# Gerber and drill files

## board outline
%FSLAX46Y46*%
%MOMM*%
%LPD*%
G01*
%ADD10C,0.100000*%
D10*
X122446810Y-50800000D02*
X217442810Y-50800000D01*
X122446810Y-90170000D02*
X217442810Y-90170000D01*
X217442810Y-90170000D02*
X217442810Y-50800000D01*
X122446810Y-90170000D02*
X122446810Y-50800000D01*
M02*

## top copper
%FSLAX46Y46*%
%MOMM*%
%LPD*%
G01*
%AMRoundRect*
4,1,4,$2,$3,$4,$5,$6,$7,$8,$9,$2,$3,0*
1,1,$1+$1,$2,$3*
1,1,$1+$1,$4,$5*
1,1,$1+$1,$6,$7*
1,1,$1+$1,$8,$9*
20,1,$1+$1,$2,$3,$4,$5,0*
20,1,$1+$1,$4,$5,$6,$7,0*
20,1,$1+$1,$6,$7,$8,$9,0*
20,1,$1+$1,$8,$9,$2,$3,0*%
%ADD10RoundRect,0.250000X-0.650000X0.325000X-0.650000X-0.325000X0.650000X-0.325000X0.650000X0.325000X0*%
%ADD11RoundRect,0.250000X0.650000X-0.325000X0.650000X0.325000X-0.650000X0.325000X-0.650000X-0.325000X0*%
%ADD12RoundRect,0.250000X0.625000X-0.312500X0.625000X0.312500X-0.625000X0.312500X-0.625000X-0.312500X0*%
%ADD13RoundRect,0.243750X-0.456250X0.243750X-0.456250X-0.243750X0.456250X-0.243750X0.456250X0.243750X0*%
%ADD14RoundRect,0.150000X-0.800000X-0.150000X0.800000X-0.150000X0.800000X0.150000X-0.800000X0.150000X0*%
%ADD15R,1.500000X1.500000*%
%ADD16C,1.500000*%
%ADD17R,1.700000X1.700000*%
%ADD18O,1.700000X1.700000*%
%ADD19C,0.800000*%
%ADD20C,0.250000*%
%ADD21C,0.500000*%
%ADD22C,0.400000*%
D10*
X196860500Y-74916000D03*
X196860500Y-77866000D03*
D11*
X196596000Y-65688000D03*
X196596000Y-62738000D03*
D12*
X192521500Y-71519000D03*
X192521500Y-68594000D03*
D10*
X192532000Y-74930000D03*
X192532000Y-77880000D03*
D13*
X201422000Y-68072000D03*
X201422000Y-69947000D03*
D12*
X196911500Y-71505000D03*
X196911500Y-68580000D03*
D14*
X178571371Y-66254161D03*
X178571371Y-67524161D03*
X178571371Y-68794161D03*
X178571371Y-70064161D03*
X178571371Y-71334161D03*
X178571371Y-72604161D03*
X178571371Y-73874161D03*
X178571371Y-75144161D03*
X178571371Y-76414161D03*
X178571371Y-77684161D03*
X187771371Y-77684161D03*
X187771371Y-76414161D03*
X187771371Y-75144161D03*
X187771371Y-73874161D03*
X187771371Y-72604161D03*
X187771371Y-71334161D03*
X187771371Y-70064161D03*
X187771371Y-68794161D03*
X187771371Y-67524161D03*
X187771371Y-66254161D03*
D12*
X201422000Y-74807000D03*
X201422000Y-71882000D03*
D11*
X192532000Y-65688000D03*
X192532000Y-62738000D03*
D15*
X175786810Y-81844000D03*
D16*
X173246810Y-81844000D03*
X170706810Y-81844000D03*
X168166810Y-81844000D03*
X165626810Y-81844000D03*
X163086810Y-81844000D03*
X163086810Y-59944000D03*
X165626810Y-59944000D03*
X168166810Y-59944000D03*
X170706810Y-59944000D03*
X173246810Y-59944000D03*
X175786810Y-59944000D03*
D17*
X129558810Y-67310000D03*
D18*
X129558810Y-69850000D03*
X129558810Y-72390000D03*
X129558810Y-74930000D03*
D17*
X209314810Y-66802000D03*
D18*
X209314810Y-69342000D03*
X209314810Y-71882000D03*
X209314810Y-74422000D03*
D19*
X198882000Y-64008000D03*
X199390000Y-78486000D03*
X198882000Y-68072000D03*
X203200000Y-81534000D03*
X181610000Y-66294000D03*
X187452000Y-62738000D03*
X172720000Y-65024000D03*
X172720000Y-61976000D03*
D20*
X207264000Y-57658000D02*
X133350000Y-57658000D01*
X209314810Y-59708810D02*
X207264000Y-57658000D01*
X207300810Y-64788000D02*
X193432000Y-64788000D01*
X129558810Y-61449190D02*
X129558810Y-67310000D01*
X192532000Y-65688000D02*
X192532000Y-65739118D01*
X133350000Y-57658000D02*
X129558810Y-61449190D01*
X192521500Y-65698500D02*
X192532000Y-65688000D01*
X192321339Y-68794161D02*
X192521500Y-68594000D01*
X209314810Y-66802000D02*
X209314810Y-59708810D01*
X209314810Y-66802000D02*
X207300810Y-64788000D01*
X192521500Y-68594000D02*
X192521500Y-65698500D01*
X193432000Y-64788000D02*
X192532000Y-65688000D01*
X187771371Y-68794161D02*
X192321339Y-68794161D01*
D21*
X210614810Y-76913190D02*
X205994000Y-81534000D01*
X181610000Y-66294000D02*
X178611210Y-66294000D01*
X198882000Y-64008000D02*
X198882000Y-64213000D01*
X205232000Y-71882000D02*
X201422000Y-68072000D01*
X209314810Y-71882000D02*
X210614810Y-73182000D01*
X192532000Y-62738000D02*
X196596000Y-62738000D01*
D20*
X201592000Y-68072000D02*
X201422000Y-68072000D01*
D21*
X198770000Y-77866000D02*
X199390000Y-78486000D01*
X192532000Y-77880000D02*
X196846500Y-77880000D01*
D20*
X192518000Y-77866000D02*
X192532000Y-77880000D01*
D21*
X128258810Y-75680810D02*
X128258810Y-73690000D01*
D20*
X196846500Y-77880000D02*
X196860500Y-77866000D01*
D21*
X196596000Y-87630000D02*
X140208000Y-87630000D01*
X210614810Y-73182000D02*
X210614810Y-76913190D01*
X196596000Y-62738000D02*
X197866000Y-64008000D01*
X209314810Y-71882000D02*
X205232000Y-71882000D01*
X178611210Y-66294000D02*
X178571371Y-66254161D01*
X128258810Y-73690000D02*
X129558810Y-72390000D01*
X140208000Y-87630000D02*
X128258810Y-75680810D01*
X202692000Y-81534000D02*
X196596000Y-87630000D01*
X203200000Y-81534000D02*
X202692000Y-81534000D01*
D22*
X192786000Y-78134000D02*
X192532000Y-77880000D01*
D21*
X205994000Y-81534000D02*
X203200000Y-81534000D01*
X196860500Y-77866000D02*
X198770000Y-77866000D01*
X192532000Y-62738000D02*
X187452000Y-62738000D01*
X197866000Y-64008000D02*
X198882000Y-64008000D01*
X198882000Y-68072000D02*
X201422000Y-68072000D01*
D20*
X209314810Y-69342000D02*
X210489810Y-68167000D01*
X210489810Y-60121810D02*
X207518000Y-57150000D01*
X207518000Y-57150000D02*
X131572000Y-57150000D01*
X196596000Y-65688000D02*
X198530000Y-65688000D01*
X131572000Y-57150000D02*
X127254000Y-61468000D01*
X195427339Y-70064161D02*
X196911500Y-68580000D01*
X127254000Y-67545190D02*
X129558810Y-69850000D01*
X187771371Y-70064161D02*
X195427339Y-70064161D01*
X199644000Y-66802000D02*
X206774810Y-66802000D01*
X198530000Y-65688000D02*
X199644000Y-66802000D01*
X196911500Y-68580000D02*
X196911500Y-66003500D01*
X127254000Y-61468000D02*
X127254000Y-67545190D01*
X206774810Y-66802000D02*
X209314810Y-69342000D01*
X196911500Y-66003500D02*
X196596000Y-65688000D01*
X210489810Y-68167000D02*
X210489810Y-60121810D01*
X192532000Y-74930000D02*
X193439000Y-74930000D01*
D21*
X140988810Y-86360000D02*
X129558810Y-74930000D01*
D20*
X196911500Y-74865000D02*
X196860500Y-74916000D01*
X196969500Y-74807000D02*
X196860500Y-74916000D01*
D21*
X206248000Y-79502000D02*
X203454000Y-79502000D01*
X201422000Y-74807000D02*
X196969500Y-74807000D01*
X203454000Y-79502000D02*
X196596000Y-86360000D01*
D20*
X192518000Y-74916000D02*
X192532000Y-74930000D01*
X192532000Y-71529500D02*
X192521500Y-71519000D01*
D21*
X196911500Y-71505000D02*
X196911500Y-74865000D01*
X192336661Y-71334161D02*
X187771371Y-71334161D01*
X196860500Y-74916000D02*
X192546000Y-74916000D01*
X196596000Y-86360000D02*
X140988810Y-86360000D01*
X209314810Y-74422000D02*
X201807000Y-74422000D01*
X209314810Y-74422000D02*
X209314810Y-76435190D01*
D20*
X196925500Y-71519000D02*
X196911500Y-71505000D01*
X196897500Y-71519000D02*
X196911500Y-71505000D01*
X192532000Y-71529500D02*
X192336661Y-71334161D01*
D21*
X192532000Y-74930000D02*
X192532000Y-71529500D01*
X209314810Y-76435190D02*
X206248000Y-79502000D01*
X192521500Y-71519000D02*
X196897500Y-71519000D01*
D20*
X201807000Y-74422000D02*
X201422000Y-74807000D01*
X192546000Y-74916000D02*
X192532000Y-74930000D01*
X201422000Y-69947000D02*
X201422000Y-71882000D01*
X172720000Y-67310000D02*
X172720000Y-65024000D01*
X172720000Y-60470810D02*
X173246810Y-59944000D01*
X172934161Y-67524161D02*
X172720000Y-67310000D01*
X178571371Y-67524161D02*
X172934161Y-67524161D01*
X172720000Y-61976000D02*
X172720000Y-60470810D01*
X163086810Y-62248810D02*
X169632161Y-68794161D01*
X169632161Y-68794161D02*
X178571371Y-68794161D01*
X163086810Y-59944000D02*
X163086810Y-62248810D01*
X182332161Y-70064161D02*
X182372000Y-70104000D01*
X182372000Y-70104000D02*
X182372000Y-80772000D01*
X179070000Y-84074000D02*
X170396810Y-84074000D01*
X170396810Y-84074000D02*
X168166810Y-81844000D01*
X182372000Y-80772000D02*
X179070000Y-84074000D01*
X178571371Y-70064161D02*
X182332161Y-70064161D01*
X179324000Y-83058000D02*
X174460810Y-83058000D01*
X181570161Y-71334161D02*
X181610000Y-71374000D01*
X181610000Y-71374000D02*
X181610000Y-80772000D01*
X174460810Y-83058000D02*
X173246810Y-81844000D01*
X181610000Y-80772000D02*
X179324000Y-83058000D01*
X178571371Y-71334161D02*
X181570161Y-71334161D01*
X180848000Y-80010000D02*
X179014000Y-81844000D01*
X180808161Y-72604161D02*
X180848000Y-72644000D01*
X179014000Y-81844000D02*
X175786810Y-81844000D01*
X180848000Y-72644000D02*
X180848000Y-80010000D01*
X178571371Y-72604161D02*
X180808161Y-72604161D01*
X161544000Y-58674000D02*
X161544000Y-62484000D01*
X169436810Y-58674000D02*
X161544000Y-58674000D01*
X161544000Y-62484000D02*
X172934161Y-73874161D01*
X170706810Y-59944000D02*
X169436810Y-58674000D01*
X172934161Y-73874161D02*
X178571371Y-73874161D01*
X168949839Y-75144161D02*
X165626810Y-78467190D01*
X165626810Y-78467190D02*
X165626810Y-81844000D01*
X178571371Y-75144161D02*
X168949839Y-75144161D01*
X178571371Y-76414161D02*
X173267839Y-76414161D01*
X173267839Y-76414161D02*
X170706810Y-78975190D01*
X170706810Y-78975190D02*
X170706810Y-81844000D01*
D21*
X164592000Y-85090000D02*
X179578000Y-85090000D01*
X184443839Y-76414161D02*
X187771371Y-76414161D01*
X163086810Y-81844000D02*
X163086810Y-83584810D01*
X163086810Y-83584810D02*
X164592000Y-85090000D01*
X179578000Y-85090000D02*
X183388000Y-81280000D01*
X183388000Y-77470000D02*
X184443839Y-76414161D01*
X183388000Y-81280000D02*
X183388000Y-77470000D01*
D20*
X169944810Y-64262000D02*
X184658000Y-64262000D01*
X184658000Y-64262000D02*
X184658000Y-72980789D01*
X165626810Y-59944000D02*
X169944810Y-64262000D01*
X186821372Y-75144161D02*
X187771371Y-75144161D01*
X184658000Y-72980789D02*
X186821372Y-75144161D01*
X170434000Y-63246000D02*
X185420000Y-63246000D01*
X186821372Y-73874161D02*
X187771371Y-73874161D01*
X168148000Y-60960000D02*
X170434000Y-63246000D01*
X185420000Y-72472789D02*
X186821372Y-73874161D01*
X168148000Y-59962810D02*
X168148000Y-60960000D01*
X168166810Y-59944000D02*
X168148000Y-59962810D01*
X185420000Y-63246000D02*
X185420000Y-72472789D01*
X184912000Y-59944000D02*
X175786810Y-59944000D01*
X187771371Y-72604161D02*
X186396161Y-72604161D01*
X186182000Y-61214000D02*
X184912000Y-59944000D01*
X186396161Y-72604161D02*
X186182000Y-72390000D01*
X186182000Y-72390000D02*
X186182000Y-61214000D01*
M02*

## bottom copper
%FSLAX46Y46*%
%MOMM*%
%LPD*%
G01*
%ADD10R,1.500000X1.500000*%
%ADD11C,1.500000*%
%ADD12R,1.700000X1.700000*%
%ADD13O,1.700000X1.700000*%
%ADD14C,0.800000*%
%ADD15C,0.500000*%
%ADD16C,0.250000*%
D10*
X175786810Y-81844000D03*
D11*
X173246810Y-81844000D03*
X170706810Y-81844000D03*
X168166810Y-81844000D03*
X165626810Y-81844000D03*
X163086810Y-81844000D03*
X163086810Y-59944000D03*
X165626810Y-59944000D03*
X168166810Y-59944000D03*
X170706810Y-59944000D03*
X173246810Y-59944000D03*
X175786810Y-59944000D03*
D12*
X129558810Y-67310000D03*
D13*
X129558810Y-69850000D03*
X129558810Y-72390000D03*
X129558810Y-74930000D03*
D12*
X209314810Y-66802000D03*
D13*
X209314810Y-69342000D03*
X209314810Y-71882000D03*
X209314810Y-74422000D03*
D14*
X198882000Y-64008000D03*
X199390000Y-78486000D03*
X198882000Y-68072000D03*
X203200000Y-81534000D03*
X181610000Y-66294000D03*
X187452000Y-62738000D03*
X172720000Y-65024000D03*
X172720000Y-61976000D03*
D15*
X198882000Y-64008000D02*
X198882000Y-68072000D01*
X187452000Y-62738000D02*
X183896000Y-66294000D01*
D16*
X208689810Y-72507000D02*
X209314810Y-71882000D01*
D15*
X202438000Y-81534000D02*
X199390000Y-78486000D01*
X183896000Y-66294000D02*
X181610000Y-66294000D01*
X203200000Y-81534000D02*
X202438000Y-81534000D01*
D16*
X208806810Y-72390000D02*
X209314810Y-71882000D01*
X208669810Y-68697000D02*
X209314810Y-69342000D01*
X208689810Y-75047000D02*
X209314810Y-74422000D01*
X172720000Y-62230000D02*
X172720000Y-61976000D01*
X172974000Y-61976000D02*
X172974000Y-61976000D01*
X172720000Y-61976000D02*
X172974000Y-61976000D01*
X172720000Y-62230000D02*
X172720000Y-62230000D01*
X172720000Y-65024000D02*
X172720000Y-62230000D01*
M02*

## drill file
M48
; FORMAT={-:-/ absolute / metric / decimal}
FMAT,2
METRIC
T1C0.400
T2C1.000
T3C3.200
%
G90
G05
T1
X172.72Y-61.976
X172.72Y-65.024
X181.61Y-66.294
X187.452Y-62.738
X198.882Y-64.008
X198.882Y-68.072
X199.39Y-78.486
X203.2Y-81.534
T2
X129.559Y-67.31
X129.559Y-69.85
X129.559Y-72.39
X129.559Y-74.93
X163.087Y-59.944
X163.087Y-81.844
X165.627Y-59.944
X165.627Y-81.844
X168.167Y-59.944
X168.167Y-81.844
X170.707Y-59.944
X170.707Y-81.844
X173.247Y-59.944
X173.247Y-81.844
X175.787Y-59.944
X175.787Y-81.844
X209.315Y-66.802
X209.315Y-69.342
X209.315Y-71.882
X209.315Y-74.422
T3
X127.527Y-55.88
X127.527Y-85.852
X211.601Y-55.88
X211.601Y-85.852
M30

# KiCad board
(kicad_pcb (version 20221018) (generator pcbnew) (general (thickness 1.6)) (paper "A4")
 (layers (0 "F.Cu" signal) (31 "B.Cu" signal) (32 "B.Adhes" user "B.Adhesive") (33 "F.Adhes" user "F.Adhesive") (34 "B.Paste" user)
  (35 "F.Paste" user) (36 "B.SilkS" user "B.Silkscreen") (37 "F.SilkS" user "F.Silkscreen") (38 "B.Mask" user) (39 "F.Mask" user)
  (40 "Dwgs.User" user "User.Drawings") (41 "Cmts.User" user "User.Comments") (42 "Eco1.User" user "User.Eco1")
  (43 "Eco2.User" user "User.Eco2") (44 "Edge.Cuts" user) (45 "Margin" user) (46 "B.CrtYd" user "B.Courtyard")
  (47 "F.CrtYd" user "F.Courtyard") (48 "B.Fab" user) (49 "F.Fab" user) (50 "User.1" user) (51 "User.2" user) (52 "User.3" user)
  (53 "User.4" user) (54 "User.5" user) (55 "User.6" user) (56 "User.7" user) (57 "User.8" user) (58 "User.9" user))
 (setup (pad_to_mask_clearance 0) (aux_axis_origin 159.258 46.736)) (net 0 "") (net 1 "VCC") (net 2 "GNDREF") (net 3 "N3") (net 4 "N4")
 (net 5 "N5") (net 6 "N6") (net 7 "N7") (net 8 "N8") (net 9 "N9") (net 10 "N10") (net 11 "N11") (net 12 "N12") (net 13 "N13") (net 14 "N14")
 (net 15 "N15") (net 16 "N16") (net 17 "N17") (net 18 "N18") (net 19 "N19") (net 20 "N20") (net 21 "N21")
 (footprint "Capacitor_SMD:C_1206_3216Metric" (layer "F.Cu") (at 196.8605 76.391 -90)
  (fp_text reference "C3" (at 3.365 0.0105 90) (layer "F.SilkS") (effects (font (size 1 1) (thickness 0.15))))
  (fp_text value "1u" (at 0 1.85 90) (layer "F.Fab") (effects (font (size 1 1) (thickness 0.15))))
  (pad "1" smd roundrect (at -1.475 0 270) (size 1.15 1.8) (layers "F.Cu" "F.Paste" "F.Mask") (roundrect_rratio 0.217391) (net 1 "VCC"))
  (pad "2" smd roundrect (at 1.475 0 270) (size 1.15 1.8) (layers "F.Cu" "F.Paste" "F.Mask") (roundrect_rratio 0.217391) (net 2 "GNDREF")))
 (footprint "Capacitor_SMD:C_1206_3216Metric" (layer "F.Cu") (at 196.596 64.213 90)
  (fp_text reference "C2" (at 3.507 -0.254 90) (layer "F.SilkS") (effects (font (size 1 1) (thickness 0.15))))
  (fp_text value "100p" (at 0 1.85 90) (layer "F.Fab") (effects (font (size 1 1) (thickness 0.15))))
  (pad "1" smd roundrect (at -1.475 0 90) (size 1.15 1.8) (layers "F.Cu" "F.Paste" "F.Mask") (roundrect_rratio 0.217391) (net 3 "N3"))
  (pad "2" smd roundrect (at 1.475 0 90) (size 1.15 1.8) (layers "F.Cu" "F.Paste" "F.Mask") (roundrect_rratio 0.217391) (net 2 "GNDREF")))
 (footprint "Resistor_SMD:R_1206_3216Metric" (layer "F.Cu") (at 192.5215 70.0565 90)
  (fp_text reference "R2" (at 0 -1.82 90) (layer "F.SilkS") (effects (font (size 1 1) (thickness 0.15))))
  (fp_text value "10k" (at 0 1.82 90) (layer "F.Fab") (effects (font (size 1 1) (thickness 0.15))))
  (pad "1" smd roundrect (at -1.4625 0 90) (size 1.125 1.75) (layers "F.Cu" "F.Paste" "F.Mask") (roundrect_rratio 0.222222) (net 1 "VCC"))
  (pad "2" smd roundrect (at 1.4625 0 90) (size 1.125 1.75) (layers "F.Cu" "F.Paste" "F.Mask") (roundrect_rratio 0.222222) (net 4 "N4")))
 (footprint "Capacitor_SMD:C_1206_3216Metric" (layer "F.Cu") (at 192.532 76.405 -90)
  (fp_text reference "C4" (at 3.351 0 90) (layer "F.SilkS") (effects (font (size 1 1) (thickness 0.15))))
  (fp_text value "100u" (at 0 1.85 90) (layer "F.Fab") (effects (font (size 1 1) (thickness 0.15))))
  (pad "1" smd roundrect (at -1.475 0 270) (size 1.15 1.8) (layers "F.Cu" "F.Paste" "F.Mask") (roundrect_rratio 0.217391) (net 1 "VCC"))
  (pad "2" smd roundrect (at 1.475 0 270) (size 1.15 1.8) (layers "F.Cu" "F.Paste" "F.Mask") (roundrect_rratio 0.217391) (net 2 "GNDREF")))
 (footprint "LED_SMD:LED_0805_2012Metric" (layer "F.Cu") (at 201.422 69.0095 -90)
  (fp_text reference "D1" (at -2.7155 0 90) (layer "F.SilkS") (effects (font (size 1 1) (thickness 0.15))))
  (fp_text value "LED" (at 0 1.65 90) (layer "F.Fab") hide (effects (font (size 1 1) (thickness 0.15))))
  (pad "1" smd roundrect (at -0.9375 0 270) (size 0.975 1.4) (layers "F.Cu" "F.Paste" "F.Mask") (roundrect_rratio 0.25) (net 2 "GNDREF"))
  (pad "2" smd roundrect (at 0.9375 0 270) (size 0.975 1.4) (layers "F.Cu" "F.Paste" "F.Mask") (roundrect_rratio 0.25) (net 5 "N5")))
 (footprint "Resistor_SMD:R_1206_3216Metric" (layer "F.Cu") (at 196.9115 70.0425 90)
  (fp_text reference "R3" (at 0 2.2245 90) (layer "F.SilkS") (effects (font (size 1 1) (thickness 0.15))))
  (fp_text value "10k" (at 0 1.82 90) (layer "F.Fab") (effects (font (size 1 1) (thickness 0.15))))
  (pad "1" smd roundrect (at -1.4625 0 90) (size 1.125 1.75) (layers "F.Cu" "F.Paste" "F.Mask") (roundrect_rratio 0.222222) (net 1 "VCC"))
  (pad "2" smd roundrect (at 1.4625 0 90) (size 1.125 1.75) (layers "F.Cu" "F.Paste" "F.Mask") (roundrect_rratio 0.222222) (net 3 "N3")))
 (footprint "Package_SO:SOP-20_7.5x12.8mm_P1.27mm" (layer "F.Cu") (at 183.171371 71.969161)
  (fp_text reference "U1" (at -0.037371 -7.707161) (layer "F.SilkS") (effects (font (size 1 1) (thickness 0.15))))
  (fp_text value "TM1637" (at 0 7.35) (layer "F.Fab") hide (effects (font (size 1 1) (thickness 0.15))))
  (pad "1" smd roundrect (at -4.6 -5.715) (size 1.9 0.6) (layers "F.Cu" "F.Paste" "F.Mask") (roundrect_rratio 0.25) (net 2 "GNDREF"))
  (pad "2" smd roundrect (at -4.6 -4.445) (size 1.9 0.6) (layers "F.Cu" "F.Paste" "F.Mask") (roundrect_rratio 0.25) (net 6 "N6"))
  (pad "3" smd roundrect (at -4.6 -3.175) (size 1.9 0.6) (layers "F.Cu" "F.Paste" "F.Mask") (roundrect_rratio 0.25) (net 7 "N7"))
  (pad "4" smd roundrect (at -4.6 -1.905) (size 1.9 0.6) (layers "F.Cu" "F.Paste" "F.Mask") (roundrect_rratio 0.25) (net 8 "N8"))
  (pad "5" smd roundrect (at -4.6 -0.635) (size 1.9 0.6) (layers "F.Cu" "F.Paste" "F.Mask") (roundrect_rratio 0.25) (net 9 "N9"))
  (pad "6" smd roundrect (at -4.6 0.635) (size 1.9 0.6) (layers "F.Cu" "F.Paste" "F.Mask") (roundrect_rratio 0.25) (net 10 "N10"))
  (pad "7" smd roundrect (at -4.6 1.905) (size 1.9 0.6) (layers "F.Cu" "F.Paste" "F.Mask") (roundrect_rratio 0.25) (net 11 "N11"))
  (pad "8" smd roundrect (at -4.6 3.175) (size 1.9 0.6) (layers "F.Cu" "F.Paste" "F.Mask") (roundrect_rratio 0.25) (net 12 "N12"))
  (pad "9" smd roundrect (at -4.6 4.445) (size 1.9 0.6) (layers "F.Cu" "F.Paste" "F.Mask") (roundrect_rratio 0.25) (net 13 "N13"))
  (pad "10" smd roundrect (at -4.6 5.715) (size 1.9 0.6) (layers "F.Cu" "F.Paste" "F.Mask") (roundrect_rratio 0.25) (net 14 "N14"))
  (pad "11" smd roundrect (at 4.6 5.715) (size 1.9 0.6) (layers "F.Cu" "F.Paste" "F.Mask") (roundrect_rratio 0.25) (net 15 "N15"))
  (pad "12" smd roundrect (at 4.6 4.445) (size 1.9 0.6) (layers "F.Cu" "F.Paste" "F.Mask") (roundrect_rratio 0.25) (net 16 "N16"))
  (pad "13" smd roundrect (at 4.6 3.175) (size 1.9 0.6) (layers "F.Cu" "F.Paste" "F.Mask") (roundrect_rratio 0.25) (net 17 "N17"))
  (pad "14" smd roundrect (at 4.6 1.905) (size 1.9 0.6) (layers "F.Cu" "F.Paste" "F.Mask") (roundrect_rratio 0.25) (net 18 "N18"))
  (pad "15" smd roundrect (at 4.6 0.635) (size 1.9 0.6) (layers "F.Cu" "F.Paste" "F.Mask") (roundrect_rratio 0.25) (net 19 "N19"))
  (pad "16" smd roundrect (at 4.6 -0.635) (size 1.9 0.6) (layers "F.Cu" "F.Paste" "F.Mask") (roundrect_rratio 0.25) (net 1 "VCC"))
  (pad "17" smd roundrect (at 4.6 -1.905) (size 1.9 0.6) (layers "F.Cu" "F.Paste" "F.Mask") (roundrect_rratio 0.25) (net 3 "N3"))
  (pad "18" smd roundrect (at 4.6 -3.175) (size 1.9 0.6) (layers "F.Cu" "F.Paste" "F.Mask") (roundrect_rratio 0.25) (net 4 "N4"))
  (pad "19" smd roundrect (at 4.6 -4.445) (size 1.9 0.6) (layers "F.Cu" "F.Paste" "F.Mask") (roundrect_rratio 0.25) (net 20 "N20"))
  (pad "20" smd roundrect (at 4.6 -5.715) (size 1.9 0.6) (layers "F.Cu" "F.Paste" "F.Mask") (roundrect_rratio 0.25) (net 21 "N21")))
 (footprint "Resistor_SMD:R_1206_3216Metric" (layer "F.Cu") (at 201.422 73.3445 90)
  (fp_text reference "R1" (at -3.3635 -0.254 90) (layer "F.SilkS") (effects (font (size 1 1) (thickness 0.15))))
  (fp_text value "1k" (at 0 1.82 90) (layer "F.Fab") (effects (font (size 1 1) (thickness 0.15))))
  (pad "1" smd roundrect (at -1.4625 0 90) (size 1.125 1.75) (layers "F.Cu" "F.Paste" "F.Mask") (roundrect_rratio 0.222222) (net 1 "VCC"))
  (pad "2" smd roundrect (at 1.4625 0 90) (size 1.125 1.75) (layers "F.Cu" "F.Paste" "F.Mask") (roundrect_rratio 0.222222) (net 5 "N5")))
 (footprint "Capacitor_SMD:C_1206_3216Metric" (layer "F.Cu") (at 192.532 64.213 90)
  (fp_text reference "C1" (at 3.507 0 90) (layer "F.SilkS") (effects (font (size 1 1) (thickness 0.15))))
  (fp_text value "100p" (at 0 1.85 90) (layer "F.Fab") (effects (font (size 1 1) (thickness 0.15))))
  (pad "1" smd roundrect (at -1.475 0 90) (size 1.15 1.8) (layers "F.Cu" "F.Paste" "F.Mask") (roundrect_rratio 0.217391) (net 4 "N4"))
  (pad "2" smd roundrect (at 1.475 0 90) (size 1.15 1.8) (layers "F.Cu" "F.Paste" "F.Mask") (roundrect_rratio 0.217391) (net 2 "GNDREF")))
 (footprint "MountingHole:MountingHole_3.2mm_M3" (layer "B.Cu") (at 211.60081 85.852 180)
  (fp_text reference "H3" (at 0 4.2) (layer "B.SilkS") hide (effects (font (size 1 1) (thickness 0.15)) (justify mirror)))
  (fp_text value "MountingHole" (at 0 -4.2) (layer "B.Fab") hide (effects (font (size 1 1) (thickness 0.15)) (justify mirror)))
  (pad "" np_thru_hole circle (at 0 0 180) (size 3.2 3.2) (drill 3.2) (layers "*.Cu" "*.Mask")))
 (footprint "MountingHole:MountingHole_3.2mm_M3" (layer "B.Cu") (at 211.60081 55.88 180)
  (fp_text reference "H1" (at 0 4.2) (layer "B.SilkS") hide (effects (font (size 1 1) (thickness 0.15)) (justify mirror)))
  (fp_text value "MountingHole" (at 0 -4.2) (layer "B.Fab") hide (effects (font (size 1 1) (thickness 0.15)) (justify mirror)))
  (pad "" np_thru_hole circle (at 0 0 180) (size 3.2 3.2) (drill 3.2) (layers "*.Cu" "*.Mask")))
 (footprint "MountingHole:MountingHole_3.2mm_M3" (layer "B.Cu") (at 127.52681 55.88 180)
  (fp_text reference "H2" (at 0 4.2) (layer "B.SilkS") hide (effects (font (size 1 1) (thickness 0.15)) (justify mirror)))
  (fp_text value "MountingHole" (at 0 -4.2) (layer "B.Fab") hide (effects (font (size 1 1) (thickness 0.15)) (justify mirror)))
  (pad "" np_thru_hole circle (at 0 0 180) (size 3.2 3.2) (drill 3.2) (layers "*.Cu" "*.Mask")))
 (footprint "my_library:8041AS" (layer "B.Cu") (at 175.78681 81.844 90)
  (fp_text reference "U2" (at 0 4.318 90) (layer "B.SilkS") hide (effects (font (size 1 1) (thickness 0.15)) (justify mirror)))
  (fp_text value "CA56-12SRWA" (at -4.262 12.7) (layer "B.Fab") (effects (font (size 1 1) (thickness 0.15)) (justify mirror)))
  (pad "1" thru_hole rect (at 0 0 90) (size 1.5 1.5) (drill 1) (layers "*.Cu" "*.Mask") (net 10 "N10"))
  (pad "2" thru_hole circle (at 0 -2.54 90) (size 1.5 1.5) (drill 1) (layers "*.Cu" "*.Mask") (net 9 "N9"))
  (pad "3" thru_hole circle (at 0 -5.08 90) (size 1.5 1.5) (drill 1) (layers "*.Cu" "*.Mask") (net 13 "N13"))
  (pad "4" thru_hole circle (at 0 -7.62 90) (size 1.5 1.5) (drill 1) (layers "*.Cu" "*.Mask") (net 8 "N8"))
  (pad "5" thru_hole circle (at 0 -10.16 90) (size 1.5 1.5) (drill 1) (layers "*.Cu" "*.Mask") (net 12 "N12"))
  (pad "6" thru_hole circle (at 0 -12.7 90) (size 1.5 1.5) (drill 1) (layers "*.Cu" "*.Mask") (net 16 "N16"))
  (pad "7" thru_hole circle (at 21.9 -12.7 90) (size 1.5 1.5) (drill 1) (layers "*.Cu" "*.Mask") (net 7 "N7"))
  (pad "8" thru_hole circle (at 21.9 -10.16 90) (size 1.5 1.5) (drill 1) (layers "*.Cu" "*.Mask") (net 17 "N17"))
  (pad "9" thru_hole circle (at 21.9 -7.62 90) (size 1.5 1.5) (drill 1) (layers "*.Cu" "*.Mask") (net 18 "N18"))
  (pad "10" thru_hole circle (at 21.9 -5.08 90) (size 1.5 1.5) (drill 1) (layers "*.Cu" "*.Mask") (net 11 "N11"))
  (pad "11" thru_hole circle (at 21.9 -2.54 90) (size 1.5 1.5) (drill 1) (layers "*.Cu" "*.Mask") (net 6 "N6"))
  (pad "12" thru_hole circle (at 21.9 0 90) (size 1.5 1.5) (drill 1) (layers "*.Cu" "*.Mask") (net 19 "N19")))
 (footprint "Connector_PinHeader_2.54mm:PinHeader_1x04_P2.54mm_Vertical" (layer "B.Cu") (at 129.55881 67.31 180)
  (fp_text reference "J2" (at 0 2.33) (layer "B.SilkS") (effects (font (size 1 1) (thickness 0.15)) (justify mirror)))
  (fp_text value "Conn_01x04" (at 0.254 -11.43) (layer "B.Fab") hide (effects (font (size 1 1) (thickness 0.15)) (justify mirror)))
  (pad "1" thru_hole rect (at 0 0 180) (size 1.7 1.7) (drill 1) (layers "*.Cu" "*.Mask") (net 4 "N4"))
  (pad "2" thru_hole oval (at 0 -2.54 180) (size 1.7 1.7) (drill 1) (layers "*.Cu" "*.Mask") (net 3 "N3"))
  (pad "3" thru_hole oval (at 0 -5.08 180) (size 1.7 1.7) (drill 1) (layers "*.Cu" "*.Mask") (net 2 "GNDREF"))
  (pad "4" thru_hole oval (at 0 -7.62 180) (size 1.7 1.7) (drill 1) (layers "*.Cu" "*.Mask") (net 1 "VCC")))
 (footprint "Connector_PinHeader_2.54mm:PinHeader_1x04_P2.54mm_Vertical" (layer "B.Cu") (at 209.31481 66.802 180)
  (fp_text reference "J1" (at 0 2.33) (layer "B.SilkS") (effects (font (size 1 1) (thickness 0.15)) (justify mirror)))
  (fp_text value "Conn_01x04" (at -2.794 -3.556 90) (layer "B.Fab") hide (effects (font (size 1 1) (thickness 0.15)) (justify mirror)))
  (pad "1" thru_hole rect (at 0 0 180) (size 1.7 1.7) (drill 1) (layers "*.Cu" "*.Mask") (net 4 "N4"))
  (pad "2" thru_hole oval (at 0 -2.54 180) (size 1.7 1.7) (drill 1) (layers "*.Cu" "*.Mask") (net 3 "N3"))
  (pad "3" thru_hole oval (at 0 -5.08 180) (size 1.7 1.7) (drill 1) (layers "*.Cu" "*.Mask") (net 2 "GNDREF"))
  (pad "4" thru_hole oval (at 0 -7.62 180) (size 1.7 1.7) (drill 1) (layers "*.Cu" "*.Mask") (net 1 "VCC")))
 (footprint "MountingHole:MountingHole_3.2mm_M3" (layer "B.Cu") (at 127.52681 85.852 180)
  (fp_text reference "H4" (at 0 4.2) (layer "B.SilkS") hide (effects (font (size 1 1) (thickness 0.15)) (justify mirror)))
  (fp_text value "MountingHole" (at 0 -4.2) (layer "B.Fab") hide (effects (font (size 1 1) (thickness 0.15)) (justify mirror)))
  (pad "" np_thru_hole circle (at 0 0 180) (size 3.2 3.2) (drill 3.2) (layers "*.Cu" "*.Mask")))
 (gr_line (start 122.44681 50.8) (end 217.44281 50.8) (stroke (width 0.1) (type default)) (layer "Edge.Cuts"))
 (gr_line (start 122.44681 90.17) (end 217.44281 90.17) (stroke (width 0.1) (type default)) (layer "Edge.Cuts"))
 (gr_line (start 217.44281 90.17) (end 217.44281 50.8) (stroke (width 0.1) (type default)) (layer "Edge.Cuts"))
 (gr_line (start 122.44681 90.17) (end 122.44681 50.8) (stroke (width 0.1) (type default)) (layer "Edge.Cuts"))
 (segment (start 207.264 57.658) (end 133.35 57.658) (width 0.25) (layer "F.Cu") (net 4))
 (segment (start 209.31481 59.70881) (end 207.264 57.658) (width 0.25) (layer "F.Cu") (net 4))
 (segment (start 207.30081 64.788) (end 193.432 64.788) (width 0.25) (layer "F.Cu") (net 4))
 (segment (start 129.55881 61.44919) (end 129.55881 67.31) (width 0.25) (layer "F.Cu") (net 4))
 (segment (start 192.532 65.688) (end 192.532 65.739118) (width 0.25) (layer "F.Cu") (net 4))
 (segment (start 133.35 57.658) (end 129.55881 61.44919) (width 0.25) (layer "F.Cu") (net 4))
 (segment (start 192.5215 65.6985) (end 192.532 65.688) (width 0.25) (layer "F.Cu") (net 4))
 (segment (start 192.321339 68.794161) (end 192.5215 68.594) (width 0.25) (layer "F.Cu") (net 4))
 (segment (start 209.31481 66.802) (end 209.31481 59.70881) (width 0.25) (layer "F.Cu") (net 4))
 (segment (start 209.31481 66.802) (end 207.30081 64.788) (width 0.25) (layer "F.Cu") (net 4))
 (segment (start 192.5215 68.594) (end 192.5215 65.6985) (width 0.25) (layer "F.Cu") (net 4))
 (segment (start 193.432 64.788) (end 192.532 65.688) (width 0.25) (layer "F.Cu") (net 4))
 (segment (start 187.771371 68.794161) (end 192.321339 68.794161) (width 0.25) (layer "F.Cu") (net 4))
 (segment (start 210.61481 76.91319) (end 205.994 81.534) (width 0.5) (layer "F.Cu") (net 2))
 (segment (start 181.61 66.294) (end 178.61121 66.294) (width 0.5) (layer "F.Cu") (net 2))
 (segment (start 198.882 64.008) (end 198.882 64.213) (width 0.5) (layer "F.Cu") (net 2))
 (segment (start 205.232 71.882) (end 201.422 68.072) (width 0.5) (layer "F.Cu") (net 2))
 (segment (start 209.31481 71.882) (end 210.61481 73.182) (width 0.5) (layer "F.Cu") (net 2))
 (segment (start 192.532 62.738) (end 196.596 62.738) (width 0.5) (layer "F.Cu") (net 2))
 (segment (start 201.592 68.072) (end 201.422 68.072) (width 0.25) (layer "F.Cu") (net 2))
 (segment (start 198.77 77.866) (end 199.39 78.486) (width 0.5) (layer "F.Cu") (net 2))
 (segment (start 192.532 77.88) (end 196.8465 77.88) (width 0.5) (layer "F.Cu") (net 2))
 (segment (start 192.518 77.866) (end 192.532 77.88) (width 0.25) (layer "F.Cu") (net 2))
 (segment (start 128.25881 75.68081) (end 128.25881 73.69) (width 0.5) (layer "F.Cu") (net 2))
 (segment (start 196.8465 77.88) (end 196.8605 77.866) (width 0.25) (layer "F.Cu") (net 2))
 (segment (start 196.596 87.63) (end 140.208 87.63) (width 0.5) (layer "F.Cu") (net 2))
 (segment (start 210.61481 73.182) (end 210.61481 76.91319) (width 0.5) (layer "F.Cu") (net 2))
 (segment (start 196.596 62.738) (end 197.866 64.008) (width 0.5) (layer "F.Cu") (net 2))
 (segment (start 209.31481 71.882) (end 205.232 71.882) (width 0.5) (layer "F.Cu") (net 2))
 (segment (start 178.61121 66.294) (end 178.571371 66.254161) (width 0.5) (layer "F.Cu") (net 2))
 (segment (start 128.25881 73.69) (end 129.55881 72.39) (width 0.5) (layer "F.Cu") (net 2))
 (segment (start 140.208 87.63) (end 128.25881 75.68081) (width 0.5) (layer "F.Cu") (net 2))
 (segment (start 202.692 81.534) (end 196.596 87.63) (width 0.5) (layer "F.Cu") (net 2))
 (segment (start 203.2 81.534) (end 202.692 81.534) (width 0.5) (layer "F.Cu") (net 2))
 (segment (start 192.786 78.134) (end 192.532 77.88) (width 0.4) (layer "F.Cu") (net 2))
 (segment (start 205.994 81.534) (end 203.2 81.534) (width 0.5) (layer "F.Cu") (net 2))
 (segment (start 196.8605 77.866) (end 198.77 77.866) (width 0.5) (layer "F.Cu") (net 2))
 (segment (start 192.532 62.738) (end 187.452 62.738) (width 0.5) (layer "F.Cu") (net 2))
 (segment (start 197.866 64.008) (end 198.882 64.008) (width 0.5) (layer "F.Cu") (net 2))
 (segment (start 198.882 68.072) (end 201.422 68.072) (width 0.5) (layer "F.Cu") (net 2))
 (via (at 198.882 64.008) (size 0.8) (drill 0.4) (layers "F.Cu" "B.Cu") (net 2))
 (via (at 199.39 78.486) (size 0.8) (drill 0.4) (layers "F.Cu" "B.Cu") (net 2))
 (via (at 198.882 68.072) (size 0.8) (drill 0.4) (layers "F.Cu" "B.Cu") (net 2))
 (via (at 203.2 81.534) (size 0.8) (drill 0.4) (layers "F.Cu" "B.Cu") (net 2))
 (via (at 181.61 66.294) (size 0.8) (drill 0.4) (layers "F.Cu" "B.Cu") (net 2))
 (via (at 187.452 62.738) (size 0.8) (drill 0.4) (layers "F.Cu" "B.Cu") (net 2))
 (segment (start 198.882 64.008) (end 198.882 68.072) (width 0.5) (layer "B.Cu") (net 2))
 (segment (start 187.452 62.738) (end 183.896 66.294) (width 0.5) (layer "B.Cu") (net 2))
 (segment (start 208.68981 72.507) (end 209.31481 71.882) (width 0.25) (layer "B.Cu") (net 2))
 (segment (start 202.438 81.534) (end 199.39 78.486) (width 0.5) (layer "B.Cu") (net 2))
 (segment (start 183.896 66.294) (end 181.61 66.294) (width 0.5) (layer "B.Cu") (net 2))
 (segment (start 203.2 81.534) (end 202.438 81.534) (width 0.5) (layer "B.Cu") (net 2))
 (segment (start 208.80681 72.39) (end 209.31481 71.882) (width 0.25) (layer "B.Cu") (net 2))
 (segment (start 209.31481 69.342) (end 210.48981 68.167) (width 0.25) (layer "F.Cu") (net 3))
 (segment (start 210.48981 60.12181) (end 207.518 57.15) (width 0.25) (layer "F.Cu") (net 3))
 (segment (start 207.518 57.15) (end 131.572 57.15) (width 0.25) (layer "F.Cu") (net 3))
 (segment (start 196.596 65.688) (end 198.53 65.688) (width 0.25) (layer "F.Cu") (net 3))
 (segment (start 131.572 57.15) (end 127.254 61.468) (width 0.25) (layer "F.Cu") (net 3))
 (segment (start 195.427339 70.064161) (end 196.9115 68.58) (width 0.25) (layer "F.Cu") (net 3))
 (segment (start 127.254 67.54519) (end 129.55881 69.85) (width 0.25) (layer "F.Cu") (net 3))
 (segment (start 187.771371 70.064161) (end 195.427339 70.064161) (width 0.25) (layer "F.Cu") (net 3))
 (segment (start 199.644 66.802) (end 206.77481 66.802) (width 0.25) (layer "F.Cu") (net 3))
 (segment (start 198.53 65.688) (end 199.644 66.802) (width 0.25) (layer "F.Cu") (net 3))
 (segment (start 196.9115 68.58) (end 196.9115 66.0035) (width 0.25) (layer "F.Cu") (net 3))
 (segment (start 127.254 61.468) (end 127.254 67.54519) (width 0.25) (layer "F.Cu") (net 3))
 (segment (start 206.77481 66.802) (end 209.31481 69.342) (width 0.25) (layer "F.Cu") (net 3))
 (segment (start 196.9115 66.0035) (end 196.596 65.688) (width 0.25) (layer "F.Cu") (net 3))
 (segment (start 210.48981 68.167) (end 210.48981 60.12181) (width 0.25) (layer "F.Cu") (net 3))
 (segment (start 208.66981 68.697) (end 209.31481 69.342) (width 0.25) (layer "B.Cu") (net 3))
 (segment (start 192.532 74.93) (end 193.439 74.93) (width 0.25) (layer "F.Cu") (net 1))
 (segment (start 140.98881 86.36) (end 129.55881 74.93) (width 0.5) (layer "F.Cu") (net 1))
 (segment (start 196.9115 74.865) (end 196.8605 74.916) (width 0.25) (layer "F.Cu") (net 1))
 (segment (start 196.9695 74.807) (end 196.8605 74.916) (width 0.25) (layer "F.Cu") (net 1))
 (segment (start 206.248 79.502) (end 203.454 79.502) (width 0.5) (layer "F.Cu") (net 1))
 (segment (start 201.422 74.807) (end 196.9695 74.807) (width 0.5) (layer "F.Cu") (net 1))
 (segment (start 203.454 79.502) (end 196.596 86.36) (width 0.5) (layer "F.Cu") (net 1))
 (segment (start 192.518 74.916) (end 192.532 74.93) (width 0.25) (layer "F.Cu") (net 1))
 (segment (start 192.532 71.5295) (end 192.5215 71.519) (width 0.25) (layer "F.Cu") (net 1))
 (segment (start 196.9115 71.505) (end 196.9115 74.865) (width 0.5) (layer "F.Cu") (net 1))
 (segment (start 192.336661 71.334161) (end 187.771371 71.334161) (width 0.5) (layer "F.Cu") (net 1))
 (segment (start 196.8605 74.916) (end 192.546 74.916) (width 0.5) (layer "F.Cu") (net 1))
 (segment (start 196.596 86.36) (end 140.98881 86.36) (width 0.5) (layer "F.Cu") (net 1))
 (segment (start 209.31481 74.422) (end 201.807 74.422) (width 0.5) (layer "F.Cu") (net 1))
 (segment (start 209.31481 74.422) (end 209.31481 76.43519) (width 0.5) (layer "F.Cu") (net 1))
 (segment (start 196.9255 71.519) (end 196.9115 71.505) (width 0.25) (layer "F.Cu") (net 1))
 (segment (start 196.8975 71.519) (end 196.9115 71.505) (width 0.25) (layer "F.Cu") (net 1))
 (segment (start 192.532 71.5295) (end 192.336661 71.334161) (width 0.25) (layer "F.Cu") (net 1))
 (segment (start 192.532 74.93) (end 192.532 71.5295) (width 0.5) (layer "F.Cu") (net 1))
 (segment (start 209.31481 76.43519) (end 206.248 79.502) (width 0.5) (layer "F.Cu") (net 1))
 (segment (start 192.5215 71.519) (end 196.8975 71.519) (width 0.5) (layer "F.Cu") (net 1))
 (segment (start 201.807 74.422) (end 201.422 74.807) (width 0.25) (layer "F.Cu") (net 1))
 (segment (start 192.546 74.916) (end 192.532 74.93) (width 0.25) (layer "F.Cu") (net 1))
 (segment (start 208.68981 75.047) (end 209.31481 74.422) (width 0.25) (layer "B.Cu") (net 1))
 (segment (start 201.422 69.947) (end 201.422 71.882) (width 0.25) (layer "F.Cu") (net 5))
 (segment (start 172.72 67.31) (end 172.72 65.024) (width 0.25) (layer "F.Cu") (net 6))
 (segment (start 172.72 60.47081) (end 173.24681 59.944) (width 0.25) (layer "F.Cu") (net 6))
 (segment (start 172.934161 67.524161) (end 172.72 67.31) (width 0.25) (layer "F.Cu") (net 6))
 (segment (start 178.571371 67.524161) (end 172.934161 67.524161) (width 0.25) (layer "F.Cu") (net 6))
 (segment (start 172.72 61.976) (end 172.72 60.47081) (width 0.25) (layer "F.Cu") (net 6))
 (via (at 172.72 65.024) (size 0.8) (drill 0.4) (layers "F.Cu" "B.Cu") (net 6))
 (via (at 172.72 61.976) (size 0.8) (drill 0.4) (layers "F.Cu" "B.Cu") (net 6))
 (segment (start 172.72 62.23) (end 172.72 61.976) (width 0.25) (layer "B.Cu") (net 6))
 (segment (start 172.974 61.976) (end 172.974 61.976) (width 0.25) (layer "B.Cu") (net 6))
 (segment (start 172.72 61.976) (end 172.974 61.976) (width 0.25) (layer "B.Cu") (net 6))
 (segment (start 172.72 62.23) (end 172.72 62.23) (width 0.25) (layer "B.Cu") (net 6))
 (segment (start 172.72 65.024) (end 172.72 62.23) (width 0.25) (layer "B.Cu") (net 6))
 (segment (start 163.08681 62.24881) (end 169.632161 68.794161) (width 0.25) (layer "F.Cu") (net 7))
 (segment (start 169.632161 68.794161) (end 178.571371 68.794161) (width 0.25) (layer "F.Cu") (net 7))
 (segment (start 163.08681 59.944) (end 163.08681 62.24881) (width 0.25) (layer "F.Cu") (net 7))
 (segment (start 182.332161 70.064161) (end 182.372 70.104) (width 0.25) (layer "F.Cu") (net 8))
 (segment (start 182.372 70.104) (end 182.372 80.772) (width 0.25) (layer "F.Cu") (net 8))
 (segment (start 179.07 84.074) (end 170.39681 84.074) (width 0.25) (layer "F.Cu") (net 8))
 (segment (start 170.39681 84.074) (end 168.16681 81.844) (width 0.25) (layer "F.Cu") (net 8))
 (segment (start 182.372 80.772) (end 179.07 84.074) (width 0.25) (layer "F.Cu") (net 8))
 (segment (start 178.571371 70.064161) (end 182.332161 70.064161) (width 0.25) (layer "F.Cu") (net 8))
 (segment (start 179.324 83.058) (end 174.46081 83.058) (width 0.25) (layer "F.Cu") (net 9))
 (segment (start 181.570161 71.334161) (end 181.61 71.374) (width 0.25) (layer "F.Cu") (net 9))
 (segment (start 181.61 71.374) (end 181.61 80.772) (width 0.25) (layer "F.Cu") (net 9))
 (segment (start 174.46081 83.058) (end 173.24681 81.844) (width 0.25) (layer "F.Cu") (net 9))
 (segment (start 181.61 80.772) (end 179.324 83.058) (width 0.25) (layer "F.Cu") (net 9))
 (segment (start 178.571371 71.334161) (end 181.570161 71.334161) (width 0.25) (layer "F.Cu") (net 9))
 (segment (start 180.848 80.01) (end 179.014 81.844) (width 0.25) (layer "F.Cu") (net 10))
 (segment (start 180.808161 72.604161) (end 180.848 72.644) (width 0.25) (layer "F.Cu") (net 10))
 (segment (start 179.014 81.844) (end 175.78681 81.844) (width 0.25) (layer "F.Cu") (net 10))
 (segment (start 180.848 72.644) (end 180.848 80.01) (width 0.25) (layer "F.Cu") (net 10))
 (segment (start 178.571371 72.604161) (end 180.808161 72.604161) (width 0.25) (layer "F.Cu") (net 10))
 (segment (start 161.544 58.674) (end 161.544 62.484) (width 0.25) (layer "F.Cu") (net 11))
 (segment (start 169.43681 58.674) (end 161.544 58.674) (width 0.25) (layer "F.Cu") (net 11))
 (segment (start 161.544 62.484) (end 172.934161 73.874161) (width 0.25) (layer "F.Cu") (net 11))
 (segment (start 170.70681 59.944) (end 169.43681 58.674) (width 0.25) (layer "F.Cu") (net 11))
 (segment (start 172.934161 73.874161) (end 178.571371 73.874161) (width 0.25) (layer "F.Cu") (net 11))
 (segment (start 168.949839 75.144161) (end 165.62681 78.46719) (width 0.25) (layer "F.Cu") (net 12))
 (segment (start 165.62681 78.46719) (end 165.62681 81.844) (width 0.25) (layer "F.Cu") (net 12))
 (segment (start 178.571371 75.144161) (end 168.949839 75.144161) (width 0.25) (layer "F.Cu") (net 12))
 (segment (start 178.571371 76.414161) (end 173.267839 76.414161) (width 0.25) (layer "F.Cu") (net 13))
 (segment (start 173.267839 76.414161) (end 170.70681 78.97519) (width 0.25) (layer "F.Cu") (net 13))
 (segment (start 170.70681 78.97519) (end 170.70681 81.844) (width 0.25) (layer "F.Cu") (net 13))
 (segment (start 164.592 85.09) (end 179.578 85.09) (width 0.5) (layer "F.Cu") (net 16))
 (segment (start 184.443839 76.414161) (end 187.771371 76.414161) (width 0.5) (layer "F.Cu") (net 16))
 (segment (start 163.08681 81.844) (end 163.08681 83.58481) (width 0.5) (layer "F.Cu") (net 16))
 (segment (start 163.08681 83.58481) (end 164.592 85.09) (width 0.5) (layer "F.Cu") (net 16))
 (segment (start 179.578 85.09) (end 183.388 81.28) (width 0.5) (layer "F.Cu") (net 16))
 (segment (start 183.388 77.47) (end 184.443839 76.414161) (width 0.5) (layer "F.Cu") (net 16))
 (segment (start 183.388 81.28) (end 183.388 77.47) (width 0.5) (layer "F.Cu") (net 16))
 (segment (start 169.94481 64.262) (end 184.658 64.262) (width 0.25) (layer "F.Cu") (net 17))
 (segment (start 184.658 64.262) (end 184.658 72.980789) (width 0.25) (layer "F.Cu") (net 17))
 (segment (start 165.62681 59.944) (end 169.94481 64.262) (width 0.25) (layer "F.Cu") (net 17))
 (segment (start 186.821372 75.144161) (end 187.771371 75.144161) (width 0.25) (layer "F.Cu") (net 17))
 (segment (start 184.658 72.980789) (end 186.821372 75.144161) (width 0.25) (layer "F.Cu") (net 17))
 (segment (start 170.434 63.246) (end 185.42 63.246) (width 0.25) (layer "F.Cu") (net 18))
 (segment (start 186.821372 73.874161) (end 187.771371 73.874161) (width 0.25) (layer "F.Cu") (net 18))
 (segment (start 168.148 60.96) (end 170.434 63.246) (width 0.25) (layer "F.Cu") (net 18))
 (segment (start 185.42 72.472789) (end 186.821372 73.874161) (width 0.25) (layer "F.Cu") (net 18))
 (segment (start 168.148 59.96281) (end 168.148 60.96) (width 0.25) (layer "F.Cu") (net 18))
 (segment (start 168.16681 59.944) (end 168.148 59.96281) (width 0.25) (layer "F.Cu") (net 18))
 (segment (start 185.42 63.246) (end 185.42 72.472789) (width 0.25) (layer "F.Cu") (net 18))
 (segment (start 184.912 59.944) (end 175.78681 59.944) (width 0.25) (layer "F.Cu") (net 19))
 (segment (start 187.771371 72.604161) (end 186.396161 72.604161) (width 0.25) (layer "F.Cu") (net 19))
 (segment (start 186.182 61.214) (end 184.912 59.944) (width 0.25) (layer "F.Cu") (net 19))
 (segment (start 186.396161 72.604161) (end 186.182 72.39) (width 0.25) (layer "F.Cu") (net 19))
 (segment (start 186.182 72.39) (end 186.182 61.214) (width 0.25) (layer "F.Cu") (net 19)))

